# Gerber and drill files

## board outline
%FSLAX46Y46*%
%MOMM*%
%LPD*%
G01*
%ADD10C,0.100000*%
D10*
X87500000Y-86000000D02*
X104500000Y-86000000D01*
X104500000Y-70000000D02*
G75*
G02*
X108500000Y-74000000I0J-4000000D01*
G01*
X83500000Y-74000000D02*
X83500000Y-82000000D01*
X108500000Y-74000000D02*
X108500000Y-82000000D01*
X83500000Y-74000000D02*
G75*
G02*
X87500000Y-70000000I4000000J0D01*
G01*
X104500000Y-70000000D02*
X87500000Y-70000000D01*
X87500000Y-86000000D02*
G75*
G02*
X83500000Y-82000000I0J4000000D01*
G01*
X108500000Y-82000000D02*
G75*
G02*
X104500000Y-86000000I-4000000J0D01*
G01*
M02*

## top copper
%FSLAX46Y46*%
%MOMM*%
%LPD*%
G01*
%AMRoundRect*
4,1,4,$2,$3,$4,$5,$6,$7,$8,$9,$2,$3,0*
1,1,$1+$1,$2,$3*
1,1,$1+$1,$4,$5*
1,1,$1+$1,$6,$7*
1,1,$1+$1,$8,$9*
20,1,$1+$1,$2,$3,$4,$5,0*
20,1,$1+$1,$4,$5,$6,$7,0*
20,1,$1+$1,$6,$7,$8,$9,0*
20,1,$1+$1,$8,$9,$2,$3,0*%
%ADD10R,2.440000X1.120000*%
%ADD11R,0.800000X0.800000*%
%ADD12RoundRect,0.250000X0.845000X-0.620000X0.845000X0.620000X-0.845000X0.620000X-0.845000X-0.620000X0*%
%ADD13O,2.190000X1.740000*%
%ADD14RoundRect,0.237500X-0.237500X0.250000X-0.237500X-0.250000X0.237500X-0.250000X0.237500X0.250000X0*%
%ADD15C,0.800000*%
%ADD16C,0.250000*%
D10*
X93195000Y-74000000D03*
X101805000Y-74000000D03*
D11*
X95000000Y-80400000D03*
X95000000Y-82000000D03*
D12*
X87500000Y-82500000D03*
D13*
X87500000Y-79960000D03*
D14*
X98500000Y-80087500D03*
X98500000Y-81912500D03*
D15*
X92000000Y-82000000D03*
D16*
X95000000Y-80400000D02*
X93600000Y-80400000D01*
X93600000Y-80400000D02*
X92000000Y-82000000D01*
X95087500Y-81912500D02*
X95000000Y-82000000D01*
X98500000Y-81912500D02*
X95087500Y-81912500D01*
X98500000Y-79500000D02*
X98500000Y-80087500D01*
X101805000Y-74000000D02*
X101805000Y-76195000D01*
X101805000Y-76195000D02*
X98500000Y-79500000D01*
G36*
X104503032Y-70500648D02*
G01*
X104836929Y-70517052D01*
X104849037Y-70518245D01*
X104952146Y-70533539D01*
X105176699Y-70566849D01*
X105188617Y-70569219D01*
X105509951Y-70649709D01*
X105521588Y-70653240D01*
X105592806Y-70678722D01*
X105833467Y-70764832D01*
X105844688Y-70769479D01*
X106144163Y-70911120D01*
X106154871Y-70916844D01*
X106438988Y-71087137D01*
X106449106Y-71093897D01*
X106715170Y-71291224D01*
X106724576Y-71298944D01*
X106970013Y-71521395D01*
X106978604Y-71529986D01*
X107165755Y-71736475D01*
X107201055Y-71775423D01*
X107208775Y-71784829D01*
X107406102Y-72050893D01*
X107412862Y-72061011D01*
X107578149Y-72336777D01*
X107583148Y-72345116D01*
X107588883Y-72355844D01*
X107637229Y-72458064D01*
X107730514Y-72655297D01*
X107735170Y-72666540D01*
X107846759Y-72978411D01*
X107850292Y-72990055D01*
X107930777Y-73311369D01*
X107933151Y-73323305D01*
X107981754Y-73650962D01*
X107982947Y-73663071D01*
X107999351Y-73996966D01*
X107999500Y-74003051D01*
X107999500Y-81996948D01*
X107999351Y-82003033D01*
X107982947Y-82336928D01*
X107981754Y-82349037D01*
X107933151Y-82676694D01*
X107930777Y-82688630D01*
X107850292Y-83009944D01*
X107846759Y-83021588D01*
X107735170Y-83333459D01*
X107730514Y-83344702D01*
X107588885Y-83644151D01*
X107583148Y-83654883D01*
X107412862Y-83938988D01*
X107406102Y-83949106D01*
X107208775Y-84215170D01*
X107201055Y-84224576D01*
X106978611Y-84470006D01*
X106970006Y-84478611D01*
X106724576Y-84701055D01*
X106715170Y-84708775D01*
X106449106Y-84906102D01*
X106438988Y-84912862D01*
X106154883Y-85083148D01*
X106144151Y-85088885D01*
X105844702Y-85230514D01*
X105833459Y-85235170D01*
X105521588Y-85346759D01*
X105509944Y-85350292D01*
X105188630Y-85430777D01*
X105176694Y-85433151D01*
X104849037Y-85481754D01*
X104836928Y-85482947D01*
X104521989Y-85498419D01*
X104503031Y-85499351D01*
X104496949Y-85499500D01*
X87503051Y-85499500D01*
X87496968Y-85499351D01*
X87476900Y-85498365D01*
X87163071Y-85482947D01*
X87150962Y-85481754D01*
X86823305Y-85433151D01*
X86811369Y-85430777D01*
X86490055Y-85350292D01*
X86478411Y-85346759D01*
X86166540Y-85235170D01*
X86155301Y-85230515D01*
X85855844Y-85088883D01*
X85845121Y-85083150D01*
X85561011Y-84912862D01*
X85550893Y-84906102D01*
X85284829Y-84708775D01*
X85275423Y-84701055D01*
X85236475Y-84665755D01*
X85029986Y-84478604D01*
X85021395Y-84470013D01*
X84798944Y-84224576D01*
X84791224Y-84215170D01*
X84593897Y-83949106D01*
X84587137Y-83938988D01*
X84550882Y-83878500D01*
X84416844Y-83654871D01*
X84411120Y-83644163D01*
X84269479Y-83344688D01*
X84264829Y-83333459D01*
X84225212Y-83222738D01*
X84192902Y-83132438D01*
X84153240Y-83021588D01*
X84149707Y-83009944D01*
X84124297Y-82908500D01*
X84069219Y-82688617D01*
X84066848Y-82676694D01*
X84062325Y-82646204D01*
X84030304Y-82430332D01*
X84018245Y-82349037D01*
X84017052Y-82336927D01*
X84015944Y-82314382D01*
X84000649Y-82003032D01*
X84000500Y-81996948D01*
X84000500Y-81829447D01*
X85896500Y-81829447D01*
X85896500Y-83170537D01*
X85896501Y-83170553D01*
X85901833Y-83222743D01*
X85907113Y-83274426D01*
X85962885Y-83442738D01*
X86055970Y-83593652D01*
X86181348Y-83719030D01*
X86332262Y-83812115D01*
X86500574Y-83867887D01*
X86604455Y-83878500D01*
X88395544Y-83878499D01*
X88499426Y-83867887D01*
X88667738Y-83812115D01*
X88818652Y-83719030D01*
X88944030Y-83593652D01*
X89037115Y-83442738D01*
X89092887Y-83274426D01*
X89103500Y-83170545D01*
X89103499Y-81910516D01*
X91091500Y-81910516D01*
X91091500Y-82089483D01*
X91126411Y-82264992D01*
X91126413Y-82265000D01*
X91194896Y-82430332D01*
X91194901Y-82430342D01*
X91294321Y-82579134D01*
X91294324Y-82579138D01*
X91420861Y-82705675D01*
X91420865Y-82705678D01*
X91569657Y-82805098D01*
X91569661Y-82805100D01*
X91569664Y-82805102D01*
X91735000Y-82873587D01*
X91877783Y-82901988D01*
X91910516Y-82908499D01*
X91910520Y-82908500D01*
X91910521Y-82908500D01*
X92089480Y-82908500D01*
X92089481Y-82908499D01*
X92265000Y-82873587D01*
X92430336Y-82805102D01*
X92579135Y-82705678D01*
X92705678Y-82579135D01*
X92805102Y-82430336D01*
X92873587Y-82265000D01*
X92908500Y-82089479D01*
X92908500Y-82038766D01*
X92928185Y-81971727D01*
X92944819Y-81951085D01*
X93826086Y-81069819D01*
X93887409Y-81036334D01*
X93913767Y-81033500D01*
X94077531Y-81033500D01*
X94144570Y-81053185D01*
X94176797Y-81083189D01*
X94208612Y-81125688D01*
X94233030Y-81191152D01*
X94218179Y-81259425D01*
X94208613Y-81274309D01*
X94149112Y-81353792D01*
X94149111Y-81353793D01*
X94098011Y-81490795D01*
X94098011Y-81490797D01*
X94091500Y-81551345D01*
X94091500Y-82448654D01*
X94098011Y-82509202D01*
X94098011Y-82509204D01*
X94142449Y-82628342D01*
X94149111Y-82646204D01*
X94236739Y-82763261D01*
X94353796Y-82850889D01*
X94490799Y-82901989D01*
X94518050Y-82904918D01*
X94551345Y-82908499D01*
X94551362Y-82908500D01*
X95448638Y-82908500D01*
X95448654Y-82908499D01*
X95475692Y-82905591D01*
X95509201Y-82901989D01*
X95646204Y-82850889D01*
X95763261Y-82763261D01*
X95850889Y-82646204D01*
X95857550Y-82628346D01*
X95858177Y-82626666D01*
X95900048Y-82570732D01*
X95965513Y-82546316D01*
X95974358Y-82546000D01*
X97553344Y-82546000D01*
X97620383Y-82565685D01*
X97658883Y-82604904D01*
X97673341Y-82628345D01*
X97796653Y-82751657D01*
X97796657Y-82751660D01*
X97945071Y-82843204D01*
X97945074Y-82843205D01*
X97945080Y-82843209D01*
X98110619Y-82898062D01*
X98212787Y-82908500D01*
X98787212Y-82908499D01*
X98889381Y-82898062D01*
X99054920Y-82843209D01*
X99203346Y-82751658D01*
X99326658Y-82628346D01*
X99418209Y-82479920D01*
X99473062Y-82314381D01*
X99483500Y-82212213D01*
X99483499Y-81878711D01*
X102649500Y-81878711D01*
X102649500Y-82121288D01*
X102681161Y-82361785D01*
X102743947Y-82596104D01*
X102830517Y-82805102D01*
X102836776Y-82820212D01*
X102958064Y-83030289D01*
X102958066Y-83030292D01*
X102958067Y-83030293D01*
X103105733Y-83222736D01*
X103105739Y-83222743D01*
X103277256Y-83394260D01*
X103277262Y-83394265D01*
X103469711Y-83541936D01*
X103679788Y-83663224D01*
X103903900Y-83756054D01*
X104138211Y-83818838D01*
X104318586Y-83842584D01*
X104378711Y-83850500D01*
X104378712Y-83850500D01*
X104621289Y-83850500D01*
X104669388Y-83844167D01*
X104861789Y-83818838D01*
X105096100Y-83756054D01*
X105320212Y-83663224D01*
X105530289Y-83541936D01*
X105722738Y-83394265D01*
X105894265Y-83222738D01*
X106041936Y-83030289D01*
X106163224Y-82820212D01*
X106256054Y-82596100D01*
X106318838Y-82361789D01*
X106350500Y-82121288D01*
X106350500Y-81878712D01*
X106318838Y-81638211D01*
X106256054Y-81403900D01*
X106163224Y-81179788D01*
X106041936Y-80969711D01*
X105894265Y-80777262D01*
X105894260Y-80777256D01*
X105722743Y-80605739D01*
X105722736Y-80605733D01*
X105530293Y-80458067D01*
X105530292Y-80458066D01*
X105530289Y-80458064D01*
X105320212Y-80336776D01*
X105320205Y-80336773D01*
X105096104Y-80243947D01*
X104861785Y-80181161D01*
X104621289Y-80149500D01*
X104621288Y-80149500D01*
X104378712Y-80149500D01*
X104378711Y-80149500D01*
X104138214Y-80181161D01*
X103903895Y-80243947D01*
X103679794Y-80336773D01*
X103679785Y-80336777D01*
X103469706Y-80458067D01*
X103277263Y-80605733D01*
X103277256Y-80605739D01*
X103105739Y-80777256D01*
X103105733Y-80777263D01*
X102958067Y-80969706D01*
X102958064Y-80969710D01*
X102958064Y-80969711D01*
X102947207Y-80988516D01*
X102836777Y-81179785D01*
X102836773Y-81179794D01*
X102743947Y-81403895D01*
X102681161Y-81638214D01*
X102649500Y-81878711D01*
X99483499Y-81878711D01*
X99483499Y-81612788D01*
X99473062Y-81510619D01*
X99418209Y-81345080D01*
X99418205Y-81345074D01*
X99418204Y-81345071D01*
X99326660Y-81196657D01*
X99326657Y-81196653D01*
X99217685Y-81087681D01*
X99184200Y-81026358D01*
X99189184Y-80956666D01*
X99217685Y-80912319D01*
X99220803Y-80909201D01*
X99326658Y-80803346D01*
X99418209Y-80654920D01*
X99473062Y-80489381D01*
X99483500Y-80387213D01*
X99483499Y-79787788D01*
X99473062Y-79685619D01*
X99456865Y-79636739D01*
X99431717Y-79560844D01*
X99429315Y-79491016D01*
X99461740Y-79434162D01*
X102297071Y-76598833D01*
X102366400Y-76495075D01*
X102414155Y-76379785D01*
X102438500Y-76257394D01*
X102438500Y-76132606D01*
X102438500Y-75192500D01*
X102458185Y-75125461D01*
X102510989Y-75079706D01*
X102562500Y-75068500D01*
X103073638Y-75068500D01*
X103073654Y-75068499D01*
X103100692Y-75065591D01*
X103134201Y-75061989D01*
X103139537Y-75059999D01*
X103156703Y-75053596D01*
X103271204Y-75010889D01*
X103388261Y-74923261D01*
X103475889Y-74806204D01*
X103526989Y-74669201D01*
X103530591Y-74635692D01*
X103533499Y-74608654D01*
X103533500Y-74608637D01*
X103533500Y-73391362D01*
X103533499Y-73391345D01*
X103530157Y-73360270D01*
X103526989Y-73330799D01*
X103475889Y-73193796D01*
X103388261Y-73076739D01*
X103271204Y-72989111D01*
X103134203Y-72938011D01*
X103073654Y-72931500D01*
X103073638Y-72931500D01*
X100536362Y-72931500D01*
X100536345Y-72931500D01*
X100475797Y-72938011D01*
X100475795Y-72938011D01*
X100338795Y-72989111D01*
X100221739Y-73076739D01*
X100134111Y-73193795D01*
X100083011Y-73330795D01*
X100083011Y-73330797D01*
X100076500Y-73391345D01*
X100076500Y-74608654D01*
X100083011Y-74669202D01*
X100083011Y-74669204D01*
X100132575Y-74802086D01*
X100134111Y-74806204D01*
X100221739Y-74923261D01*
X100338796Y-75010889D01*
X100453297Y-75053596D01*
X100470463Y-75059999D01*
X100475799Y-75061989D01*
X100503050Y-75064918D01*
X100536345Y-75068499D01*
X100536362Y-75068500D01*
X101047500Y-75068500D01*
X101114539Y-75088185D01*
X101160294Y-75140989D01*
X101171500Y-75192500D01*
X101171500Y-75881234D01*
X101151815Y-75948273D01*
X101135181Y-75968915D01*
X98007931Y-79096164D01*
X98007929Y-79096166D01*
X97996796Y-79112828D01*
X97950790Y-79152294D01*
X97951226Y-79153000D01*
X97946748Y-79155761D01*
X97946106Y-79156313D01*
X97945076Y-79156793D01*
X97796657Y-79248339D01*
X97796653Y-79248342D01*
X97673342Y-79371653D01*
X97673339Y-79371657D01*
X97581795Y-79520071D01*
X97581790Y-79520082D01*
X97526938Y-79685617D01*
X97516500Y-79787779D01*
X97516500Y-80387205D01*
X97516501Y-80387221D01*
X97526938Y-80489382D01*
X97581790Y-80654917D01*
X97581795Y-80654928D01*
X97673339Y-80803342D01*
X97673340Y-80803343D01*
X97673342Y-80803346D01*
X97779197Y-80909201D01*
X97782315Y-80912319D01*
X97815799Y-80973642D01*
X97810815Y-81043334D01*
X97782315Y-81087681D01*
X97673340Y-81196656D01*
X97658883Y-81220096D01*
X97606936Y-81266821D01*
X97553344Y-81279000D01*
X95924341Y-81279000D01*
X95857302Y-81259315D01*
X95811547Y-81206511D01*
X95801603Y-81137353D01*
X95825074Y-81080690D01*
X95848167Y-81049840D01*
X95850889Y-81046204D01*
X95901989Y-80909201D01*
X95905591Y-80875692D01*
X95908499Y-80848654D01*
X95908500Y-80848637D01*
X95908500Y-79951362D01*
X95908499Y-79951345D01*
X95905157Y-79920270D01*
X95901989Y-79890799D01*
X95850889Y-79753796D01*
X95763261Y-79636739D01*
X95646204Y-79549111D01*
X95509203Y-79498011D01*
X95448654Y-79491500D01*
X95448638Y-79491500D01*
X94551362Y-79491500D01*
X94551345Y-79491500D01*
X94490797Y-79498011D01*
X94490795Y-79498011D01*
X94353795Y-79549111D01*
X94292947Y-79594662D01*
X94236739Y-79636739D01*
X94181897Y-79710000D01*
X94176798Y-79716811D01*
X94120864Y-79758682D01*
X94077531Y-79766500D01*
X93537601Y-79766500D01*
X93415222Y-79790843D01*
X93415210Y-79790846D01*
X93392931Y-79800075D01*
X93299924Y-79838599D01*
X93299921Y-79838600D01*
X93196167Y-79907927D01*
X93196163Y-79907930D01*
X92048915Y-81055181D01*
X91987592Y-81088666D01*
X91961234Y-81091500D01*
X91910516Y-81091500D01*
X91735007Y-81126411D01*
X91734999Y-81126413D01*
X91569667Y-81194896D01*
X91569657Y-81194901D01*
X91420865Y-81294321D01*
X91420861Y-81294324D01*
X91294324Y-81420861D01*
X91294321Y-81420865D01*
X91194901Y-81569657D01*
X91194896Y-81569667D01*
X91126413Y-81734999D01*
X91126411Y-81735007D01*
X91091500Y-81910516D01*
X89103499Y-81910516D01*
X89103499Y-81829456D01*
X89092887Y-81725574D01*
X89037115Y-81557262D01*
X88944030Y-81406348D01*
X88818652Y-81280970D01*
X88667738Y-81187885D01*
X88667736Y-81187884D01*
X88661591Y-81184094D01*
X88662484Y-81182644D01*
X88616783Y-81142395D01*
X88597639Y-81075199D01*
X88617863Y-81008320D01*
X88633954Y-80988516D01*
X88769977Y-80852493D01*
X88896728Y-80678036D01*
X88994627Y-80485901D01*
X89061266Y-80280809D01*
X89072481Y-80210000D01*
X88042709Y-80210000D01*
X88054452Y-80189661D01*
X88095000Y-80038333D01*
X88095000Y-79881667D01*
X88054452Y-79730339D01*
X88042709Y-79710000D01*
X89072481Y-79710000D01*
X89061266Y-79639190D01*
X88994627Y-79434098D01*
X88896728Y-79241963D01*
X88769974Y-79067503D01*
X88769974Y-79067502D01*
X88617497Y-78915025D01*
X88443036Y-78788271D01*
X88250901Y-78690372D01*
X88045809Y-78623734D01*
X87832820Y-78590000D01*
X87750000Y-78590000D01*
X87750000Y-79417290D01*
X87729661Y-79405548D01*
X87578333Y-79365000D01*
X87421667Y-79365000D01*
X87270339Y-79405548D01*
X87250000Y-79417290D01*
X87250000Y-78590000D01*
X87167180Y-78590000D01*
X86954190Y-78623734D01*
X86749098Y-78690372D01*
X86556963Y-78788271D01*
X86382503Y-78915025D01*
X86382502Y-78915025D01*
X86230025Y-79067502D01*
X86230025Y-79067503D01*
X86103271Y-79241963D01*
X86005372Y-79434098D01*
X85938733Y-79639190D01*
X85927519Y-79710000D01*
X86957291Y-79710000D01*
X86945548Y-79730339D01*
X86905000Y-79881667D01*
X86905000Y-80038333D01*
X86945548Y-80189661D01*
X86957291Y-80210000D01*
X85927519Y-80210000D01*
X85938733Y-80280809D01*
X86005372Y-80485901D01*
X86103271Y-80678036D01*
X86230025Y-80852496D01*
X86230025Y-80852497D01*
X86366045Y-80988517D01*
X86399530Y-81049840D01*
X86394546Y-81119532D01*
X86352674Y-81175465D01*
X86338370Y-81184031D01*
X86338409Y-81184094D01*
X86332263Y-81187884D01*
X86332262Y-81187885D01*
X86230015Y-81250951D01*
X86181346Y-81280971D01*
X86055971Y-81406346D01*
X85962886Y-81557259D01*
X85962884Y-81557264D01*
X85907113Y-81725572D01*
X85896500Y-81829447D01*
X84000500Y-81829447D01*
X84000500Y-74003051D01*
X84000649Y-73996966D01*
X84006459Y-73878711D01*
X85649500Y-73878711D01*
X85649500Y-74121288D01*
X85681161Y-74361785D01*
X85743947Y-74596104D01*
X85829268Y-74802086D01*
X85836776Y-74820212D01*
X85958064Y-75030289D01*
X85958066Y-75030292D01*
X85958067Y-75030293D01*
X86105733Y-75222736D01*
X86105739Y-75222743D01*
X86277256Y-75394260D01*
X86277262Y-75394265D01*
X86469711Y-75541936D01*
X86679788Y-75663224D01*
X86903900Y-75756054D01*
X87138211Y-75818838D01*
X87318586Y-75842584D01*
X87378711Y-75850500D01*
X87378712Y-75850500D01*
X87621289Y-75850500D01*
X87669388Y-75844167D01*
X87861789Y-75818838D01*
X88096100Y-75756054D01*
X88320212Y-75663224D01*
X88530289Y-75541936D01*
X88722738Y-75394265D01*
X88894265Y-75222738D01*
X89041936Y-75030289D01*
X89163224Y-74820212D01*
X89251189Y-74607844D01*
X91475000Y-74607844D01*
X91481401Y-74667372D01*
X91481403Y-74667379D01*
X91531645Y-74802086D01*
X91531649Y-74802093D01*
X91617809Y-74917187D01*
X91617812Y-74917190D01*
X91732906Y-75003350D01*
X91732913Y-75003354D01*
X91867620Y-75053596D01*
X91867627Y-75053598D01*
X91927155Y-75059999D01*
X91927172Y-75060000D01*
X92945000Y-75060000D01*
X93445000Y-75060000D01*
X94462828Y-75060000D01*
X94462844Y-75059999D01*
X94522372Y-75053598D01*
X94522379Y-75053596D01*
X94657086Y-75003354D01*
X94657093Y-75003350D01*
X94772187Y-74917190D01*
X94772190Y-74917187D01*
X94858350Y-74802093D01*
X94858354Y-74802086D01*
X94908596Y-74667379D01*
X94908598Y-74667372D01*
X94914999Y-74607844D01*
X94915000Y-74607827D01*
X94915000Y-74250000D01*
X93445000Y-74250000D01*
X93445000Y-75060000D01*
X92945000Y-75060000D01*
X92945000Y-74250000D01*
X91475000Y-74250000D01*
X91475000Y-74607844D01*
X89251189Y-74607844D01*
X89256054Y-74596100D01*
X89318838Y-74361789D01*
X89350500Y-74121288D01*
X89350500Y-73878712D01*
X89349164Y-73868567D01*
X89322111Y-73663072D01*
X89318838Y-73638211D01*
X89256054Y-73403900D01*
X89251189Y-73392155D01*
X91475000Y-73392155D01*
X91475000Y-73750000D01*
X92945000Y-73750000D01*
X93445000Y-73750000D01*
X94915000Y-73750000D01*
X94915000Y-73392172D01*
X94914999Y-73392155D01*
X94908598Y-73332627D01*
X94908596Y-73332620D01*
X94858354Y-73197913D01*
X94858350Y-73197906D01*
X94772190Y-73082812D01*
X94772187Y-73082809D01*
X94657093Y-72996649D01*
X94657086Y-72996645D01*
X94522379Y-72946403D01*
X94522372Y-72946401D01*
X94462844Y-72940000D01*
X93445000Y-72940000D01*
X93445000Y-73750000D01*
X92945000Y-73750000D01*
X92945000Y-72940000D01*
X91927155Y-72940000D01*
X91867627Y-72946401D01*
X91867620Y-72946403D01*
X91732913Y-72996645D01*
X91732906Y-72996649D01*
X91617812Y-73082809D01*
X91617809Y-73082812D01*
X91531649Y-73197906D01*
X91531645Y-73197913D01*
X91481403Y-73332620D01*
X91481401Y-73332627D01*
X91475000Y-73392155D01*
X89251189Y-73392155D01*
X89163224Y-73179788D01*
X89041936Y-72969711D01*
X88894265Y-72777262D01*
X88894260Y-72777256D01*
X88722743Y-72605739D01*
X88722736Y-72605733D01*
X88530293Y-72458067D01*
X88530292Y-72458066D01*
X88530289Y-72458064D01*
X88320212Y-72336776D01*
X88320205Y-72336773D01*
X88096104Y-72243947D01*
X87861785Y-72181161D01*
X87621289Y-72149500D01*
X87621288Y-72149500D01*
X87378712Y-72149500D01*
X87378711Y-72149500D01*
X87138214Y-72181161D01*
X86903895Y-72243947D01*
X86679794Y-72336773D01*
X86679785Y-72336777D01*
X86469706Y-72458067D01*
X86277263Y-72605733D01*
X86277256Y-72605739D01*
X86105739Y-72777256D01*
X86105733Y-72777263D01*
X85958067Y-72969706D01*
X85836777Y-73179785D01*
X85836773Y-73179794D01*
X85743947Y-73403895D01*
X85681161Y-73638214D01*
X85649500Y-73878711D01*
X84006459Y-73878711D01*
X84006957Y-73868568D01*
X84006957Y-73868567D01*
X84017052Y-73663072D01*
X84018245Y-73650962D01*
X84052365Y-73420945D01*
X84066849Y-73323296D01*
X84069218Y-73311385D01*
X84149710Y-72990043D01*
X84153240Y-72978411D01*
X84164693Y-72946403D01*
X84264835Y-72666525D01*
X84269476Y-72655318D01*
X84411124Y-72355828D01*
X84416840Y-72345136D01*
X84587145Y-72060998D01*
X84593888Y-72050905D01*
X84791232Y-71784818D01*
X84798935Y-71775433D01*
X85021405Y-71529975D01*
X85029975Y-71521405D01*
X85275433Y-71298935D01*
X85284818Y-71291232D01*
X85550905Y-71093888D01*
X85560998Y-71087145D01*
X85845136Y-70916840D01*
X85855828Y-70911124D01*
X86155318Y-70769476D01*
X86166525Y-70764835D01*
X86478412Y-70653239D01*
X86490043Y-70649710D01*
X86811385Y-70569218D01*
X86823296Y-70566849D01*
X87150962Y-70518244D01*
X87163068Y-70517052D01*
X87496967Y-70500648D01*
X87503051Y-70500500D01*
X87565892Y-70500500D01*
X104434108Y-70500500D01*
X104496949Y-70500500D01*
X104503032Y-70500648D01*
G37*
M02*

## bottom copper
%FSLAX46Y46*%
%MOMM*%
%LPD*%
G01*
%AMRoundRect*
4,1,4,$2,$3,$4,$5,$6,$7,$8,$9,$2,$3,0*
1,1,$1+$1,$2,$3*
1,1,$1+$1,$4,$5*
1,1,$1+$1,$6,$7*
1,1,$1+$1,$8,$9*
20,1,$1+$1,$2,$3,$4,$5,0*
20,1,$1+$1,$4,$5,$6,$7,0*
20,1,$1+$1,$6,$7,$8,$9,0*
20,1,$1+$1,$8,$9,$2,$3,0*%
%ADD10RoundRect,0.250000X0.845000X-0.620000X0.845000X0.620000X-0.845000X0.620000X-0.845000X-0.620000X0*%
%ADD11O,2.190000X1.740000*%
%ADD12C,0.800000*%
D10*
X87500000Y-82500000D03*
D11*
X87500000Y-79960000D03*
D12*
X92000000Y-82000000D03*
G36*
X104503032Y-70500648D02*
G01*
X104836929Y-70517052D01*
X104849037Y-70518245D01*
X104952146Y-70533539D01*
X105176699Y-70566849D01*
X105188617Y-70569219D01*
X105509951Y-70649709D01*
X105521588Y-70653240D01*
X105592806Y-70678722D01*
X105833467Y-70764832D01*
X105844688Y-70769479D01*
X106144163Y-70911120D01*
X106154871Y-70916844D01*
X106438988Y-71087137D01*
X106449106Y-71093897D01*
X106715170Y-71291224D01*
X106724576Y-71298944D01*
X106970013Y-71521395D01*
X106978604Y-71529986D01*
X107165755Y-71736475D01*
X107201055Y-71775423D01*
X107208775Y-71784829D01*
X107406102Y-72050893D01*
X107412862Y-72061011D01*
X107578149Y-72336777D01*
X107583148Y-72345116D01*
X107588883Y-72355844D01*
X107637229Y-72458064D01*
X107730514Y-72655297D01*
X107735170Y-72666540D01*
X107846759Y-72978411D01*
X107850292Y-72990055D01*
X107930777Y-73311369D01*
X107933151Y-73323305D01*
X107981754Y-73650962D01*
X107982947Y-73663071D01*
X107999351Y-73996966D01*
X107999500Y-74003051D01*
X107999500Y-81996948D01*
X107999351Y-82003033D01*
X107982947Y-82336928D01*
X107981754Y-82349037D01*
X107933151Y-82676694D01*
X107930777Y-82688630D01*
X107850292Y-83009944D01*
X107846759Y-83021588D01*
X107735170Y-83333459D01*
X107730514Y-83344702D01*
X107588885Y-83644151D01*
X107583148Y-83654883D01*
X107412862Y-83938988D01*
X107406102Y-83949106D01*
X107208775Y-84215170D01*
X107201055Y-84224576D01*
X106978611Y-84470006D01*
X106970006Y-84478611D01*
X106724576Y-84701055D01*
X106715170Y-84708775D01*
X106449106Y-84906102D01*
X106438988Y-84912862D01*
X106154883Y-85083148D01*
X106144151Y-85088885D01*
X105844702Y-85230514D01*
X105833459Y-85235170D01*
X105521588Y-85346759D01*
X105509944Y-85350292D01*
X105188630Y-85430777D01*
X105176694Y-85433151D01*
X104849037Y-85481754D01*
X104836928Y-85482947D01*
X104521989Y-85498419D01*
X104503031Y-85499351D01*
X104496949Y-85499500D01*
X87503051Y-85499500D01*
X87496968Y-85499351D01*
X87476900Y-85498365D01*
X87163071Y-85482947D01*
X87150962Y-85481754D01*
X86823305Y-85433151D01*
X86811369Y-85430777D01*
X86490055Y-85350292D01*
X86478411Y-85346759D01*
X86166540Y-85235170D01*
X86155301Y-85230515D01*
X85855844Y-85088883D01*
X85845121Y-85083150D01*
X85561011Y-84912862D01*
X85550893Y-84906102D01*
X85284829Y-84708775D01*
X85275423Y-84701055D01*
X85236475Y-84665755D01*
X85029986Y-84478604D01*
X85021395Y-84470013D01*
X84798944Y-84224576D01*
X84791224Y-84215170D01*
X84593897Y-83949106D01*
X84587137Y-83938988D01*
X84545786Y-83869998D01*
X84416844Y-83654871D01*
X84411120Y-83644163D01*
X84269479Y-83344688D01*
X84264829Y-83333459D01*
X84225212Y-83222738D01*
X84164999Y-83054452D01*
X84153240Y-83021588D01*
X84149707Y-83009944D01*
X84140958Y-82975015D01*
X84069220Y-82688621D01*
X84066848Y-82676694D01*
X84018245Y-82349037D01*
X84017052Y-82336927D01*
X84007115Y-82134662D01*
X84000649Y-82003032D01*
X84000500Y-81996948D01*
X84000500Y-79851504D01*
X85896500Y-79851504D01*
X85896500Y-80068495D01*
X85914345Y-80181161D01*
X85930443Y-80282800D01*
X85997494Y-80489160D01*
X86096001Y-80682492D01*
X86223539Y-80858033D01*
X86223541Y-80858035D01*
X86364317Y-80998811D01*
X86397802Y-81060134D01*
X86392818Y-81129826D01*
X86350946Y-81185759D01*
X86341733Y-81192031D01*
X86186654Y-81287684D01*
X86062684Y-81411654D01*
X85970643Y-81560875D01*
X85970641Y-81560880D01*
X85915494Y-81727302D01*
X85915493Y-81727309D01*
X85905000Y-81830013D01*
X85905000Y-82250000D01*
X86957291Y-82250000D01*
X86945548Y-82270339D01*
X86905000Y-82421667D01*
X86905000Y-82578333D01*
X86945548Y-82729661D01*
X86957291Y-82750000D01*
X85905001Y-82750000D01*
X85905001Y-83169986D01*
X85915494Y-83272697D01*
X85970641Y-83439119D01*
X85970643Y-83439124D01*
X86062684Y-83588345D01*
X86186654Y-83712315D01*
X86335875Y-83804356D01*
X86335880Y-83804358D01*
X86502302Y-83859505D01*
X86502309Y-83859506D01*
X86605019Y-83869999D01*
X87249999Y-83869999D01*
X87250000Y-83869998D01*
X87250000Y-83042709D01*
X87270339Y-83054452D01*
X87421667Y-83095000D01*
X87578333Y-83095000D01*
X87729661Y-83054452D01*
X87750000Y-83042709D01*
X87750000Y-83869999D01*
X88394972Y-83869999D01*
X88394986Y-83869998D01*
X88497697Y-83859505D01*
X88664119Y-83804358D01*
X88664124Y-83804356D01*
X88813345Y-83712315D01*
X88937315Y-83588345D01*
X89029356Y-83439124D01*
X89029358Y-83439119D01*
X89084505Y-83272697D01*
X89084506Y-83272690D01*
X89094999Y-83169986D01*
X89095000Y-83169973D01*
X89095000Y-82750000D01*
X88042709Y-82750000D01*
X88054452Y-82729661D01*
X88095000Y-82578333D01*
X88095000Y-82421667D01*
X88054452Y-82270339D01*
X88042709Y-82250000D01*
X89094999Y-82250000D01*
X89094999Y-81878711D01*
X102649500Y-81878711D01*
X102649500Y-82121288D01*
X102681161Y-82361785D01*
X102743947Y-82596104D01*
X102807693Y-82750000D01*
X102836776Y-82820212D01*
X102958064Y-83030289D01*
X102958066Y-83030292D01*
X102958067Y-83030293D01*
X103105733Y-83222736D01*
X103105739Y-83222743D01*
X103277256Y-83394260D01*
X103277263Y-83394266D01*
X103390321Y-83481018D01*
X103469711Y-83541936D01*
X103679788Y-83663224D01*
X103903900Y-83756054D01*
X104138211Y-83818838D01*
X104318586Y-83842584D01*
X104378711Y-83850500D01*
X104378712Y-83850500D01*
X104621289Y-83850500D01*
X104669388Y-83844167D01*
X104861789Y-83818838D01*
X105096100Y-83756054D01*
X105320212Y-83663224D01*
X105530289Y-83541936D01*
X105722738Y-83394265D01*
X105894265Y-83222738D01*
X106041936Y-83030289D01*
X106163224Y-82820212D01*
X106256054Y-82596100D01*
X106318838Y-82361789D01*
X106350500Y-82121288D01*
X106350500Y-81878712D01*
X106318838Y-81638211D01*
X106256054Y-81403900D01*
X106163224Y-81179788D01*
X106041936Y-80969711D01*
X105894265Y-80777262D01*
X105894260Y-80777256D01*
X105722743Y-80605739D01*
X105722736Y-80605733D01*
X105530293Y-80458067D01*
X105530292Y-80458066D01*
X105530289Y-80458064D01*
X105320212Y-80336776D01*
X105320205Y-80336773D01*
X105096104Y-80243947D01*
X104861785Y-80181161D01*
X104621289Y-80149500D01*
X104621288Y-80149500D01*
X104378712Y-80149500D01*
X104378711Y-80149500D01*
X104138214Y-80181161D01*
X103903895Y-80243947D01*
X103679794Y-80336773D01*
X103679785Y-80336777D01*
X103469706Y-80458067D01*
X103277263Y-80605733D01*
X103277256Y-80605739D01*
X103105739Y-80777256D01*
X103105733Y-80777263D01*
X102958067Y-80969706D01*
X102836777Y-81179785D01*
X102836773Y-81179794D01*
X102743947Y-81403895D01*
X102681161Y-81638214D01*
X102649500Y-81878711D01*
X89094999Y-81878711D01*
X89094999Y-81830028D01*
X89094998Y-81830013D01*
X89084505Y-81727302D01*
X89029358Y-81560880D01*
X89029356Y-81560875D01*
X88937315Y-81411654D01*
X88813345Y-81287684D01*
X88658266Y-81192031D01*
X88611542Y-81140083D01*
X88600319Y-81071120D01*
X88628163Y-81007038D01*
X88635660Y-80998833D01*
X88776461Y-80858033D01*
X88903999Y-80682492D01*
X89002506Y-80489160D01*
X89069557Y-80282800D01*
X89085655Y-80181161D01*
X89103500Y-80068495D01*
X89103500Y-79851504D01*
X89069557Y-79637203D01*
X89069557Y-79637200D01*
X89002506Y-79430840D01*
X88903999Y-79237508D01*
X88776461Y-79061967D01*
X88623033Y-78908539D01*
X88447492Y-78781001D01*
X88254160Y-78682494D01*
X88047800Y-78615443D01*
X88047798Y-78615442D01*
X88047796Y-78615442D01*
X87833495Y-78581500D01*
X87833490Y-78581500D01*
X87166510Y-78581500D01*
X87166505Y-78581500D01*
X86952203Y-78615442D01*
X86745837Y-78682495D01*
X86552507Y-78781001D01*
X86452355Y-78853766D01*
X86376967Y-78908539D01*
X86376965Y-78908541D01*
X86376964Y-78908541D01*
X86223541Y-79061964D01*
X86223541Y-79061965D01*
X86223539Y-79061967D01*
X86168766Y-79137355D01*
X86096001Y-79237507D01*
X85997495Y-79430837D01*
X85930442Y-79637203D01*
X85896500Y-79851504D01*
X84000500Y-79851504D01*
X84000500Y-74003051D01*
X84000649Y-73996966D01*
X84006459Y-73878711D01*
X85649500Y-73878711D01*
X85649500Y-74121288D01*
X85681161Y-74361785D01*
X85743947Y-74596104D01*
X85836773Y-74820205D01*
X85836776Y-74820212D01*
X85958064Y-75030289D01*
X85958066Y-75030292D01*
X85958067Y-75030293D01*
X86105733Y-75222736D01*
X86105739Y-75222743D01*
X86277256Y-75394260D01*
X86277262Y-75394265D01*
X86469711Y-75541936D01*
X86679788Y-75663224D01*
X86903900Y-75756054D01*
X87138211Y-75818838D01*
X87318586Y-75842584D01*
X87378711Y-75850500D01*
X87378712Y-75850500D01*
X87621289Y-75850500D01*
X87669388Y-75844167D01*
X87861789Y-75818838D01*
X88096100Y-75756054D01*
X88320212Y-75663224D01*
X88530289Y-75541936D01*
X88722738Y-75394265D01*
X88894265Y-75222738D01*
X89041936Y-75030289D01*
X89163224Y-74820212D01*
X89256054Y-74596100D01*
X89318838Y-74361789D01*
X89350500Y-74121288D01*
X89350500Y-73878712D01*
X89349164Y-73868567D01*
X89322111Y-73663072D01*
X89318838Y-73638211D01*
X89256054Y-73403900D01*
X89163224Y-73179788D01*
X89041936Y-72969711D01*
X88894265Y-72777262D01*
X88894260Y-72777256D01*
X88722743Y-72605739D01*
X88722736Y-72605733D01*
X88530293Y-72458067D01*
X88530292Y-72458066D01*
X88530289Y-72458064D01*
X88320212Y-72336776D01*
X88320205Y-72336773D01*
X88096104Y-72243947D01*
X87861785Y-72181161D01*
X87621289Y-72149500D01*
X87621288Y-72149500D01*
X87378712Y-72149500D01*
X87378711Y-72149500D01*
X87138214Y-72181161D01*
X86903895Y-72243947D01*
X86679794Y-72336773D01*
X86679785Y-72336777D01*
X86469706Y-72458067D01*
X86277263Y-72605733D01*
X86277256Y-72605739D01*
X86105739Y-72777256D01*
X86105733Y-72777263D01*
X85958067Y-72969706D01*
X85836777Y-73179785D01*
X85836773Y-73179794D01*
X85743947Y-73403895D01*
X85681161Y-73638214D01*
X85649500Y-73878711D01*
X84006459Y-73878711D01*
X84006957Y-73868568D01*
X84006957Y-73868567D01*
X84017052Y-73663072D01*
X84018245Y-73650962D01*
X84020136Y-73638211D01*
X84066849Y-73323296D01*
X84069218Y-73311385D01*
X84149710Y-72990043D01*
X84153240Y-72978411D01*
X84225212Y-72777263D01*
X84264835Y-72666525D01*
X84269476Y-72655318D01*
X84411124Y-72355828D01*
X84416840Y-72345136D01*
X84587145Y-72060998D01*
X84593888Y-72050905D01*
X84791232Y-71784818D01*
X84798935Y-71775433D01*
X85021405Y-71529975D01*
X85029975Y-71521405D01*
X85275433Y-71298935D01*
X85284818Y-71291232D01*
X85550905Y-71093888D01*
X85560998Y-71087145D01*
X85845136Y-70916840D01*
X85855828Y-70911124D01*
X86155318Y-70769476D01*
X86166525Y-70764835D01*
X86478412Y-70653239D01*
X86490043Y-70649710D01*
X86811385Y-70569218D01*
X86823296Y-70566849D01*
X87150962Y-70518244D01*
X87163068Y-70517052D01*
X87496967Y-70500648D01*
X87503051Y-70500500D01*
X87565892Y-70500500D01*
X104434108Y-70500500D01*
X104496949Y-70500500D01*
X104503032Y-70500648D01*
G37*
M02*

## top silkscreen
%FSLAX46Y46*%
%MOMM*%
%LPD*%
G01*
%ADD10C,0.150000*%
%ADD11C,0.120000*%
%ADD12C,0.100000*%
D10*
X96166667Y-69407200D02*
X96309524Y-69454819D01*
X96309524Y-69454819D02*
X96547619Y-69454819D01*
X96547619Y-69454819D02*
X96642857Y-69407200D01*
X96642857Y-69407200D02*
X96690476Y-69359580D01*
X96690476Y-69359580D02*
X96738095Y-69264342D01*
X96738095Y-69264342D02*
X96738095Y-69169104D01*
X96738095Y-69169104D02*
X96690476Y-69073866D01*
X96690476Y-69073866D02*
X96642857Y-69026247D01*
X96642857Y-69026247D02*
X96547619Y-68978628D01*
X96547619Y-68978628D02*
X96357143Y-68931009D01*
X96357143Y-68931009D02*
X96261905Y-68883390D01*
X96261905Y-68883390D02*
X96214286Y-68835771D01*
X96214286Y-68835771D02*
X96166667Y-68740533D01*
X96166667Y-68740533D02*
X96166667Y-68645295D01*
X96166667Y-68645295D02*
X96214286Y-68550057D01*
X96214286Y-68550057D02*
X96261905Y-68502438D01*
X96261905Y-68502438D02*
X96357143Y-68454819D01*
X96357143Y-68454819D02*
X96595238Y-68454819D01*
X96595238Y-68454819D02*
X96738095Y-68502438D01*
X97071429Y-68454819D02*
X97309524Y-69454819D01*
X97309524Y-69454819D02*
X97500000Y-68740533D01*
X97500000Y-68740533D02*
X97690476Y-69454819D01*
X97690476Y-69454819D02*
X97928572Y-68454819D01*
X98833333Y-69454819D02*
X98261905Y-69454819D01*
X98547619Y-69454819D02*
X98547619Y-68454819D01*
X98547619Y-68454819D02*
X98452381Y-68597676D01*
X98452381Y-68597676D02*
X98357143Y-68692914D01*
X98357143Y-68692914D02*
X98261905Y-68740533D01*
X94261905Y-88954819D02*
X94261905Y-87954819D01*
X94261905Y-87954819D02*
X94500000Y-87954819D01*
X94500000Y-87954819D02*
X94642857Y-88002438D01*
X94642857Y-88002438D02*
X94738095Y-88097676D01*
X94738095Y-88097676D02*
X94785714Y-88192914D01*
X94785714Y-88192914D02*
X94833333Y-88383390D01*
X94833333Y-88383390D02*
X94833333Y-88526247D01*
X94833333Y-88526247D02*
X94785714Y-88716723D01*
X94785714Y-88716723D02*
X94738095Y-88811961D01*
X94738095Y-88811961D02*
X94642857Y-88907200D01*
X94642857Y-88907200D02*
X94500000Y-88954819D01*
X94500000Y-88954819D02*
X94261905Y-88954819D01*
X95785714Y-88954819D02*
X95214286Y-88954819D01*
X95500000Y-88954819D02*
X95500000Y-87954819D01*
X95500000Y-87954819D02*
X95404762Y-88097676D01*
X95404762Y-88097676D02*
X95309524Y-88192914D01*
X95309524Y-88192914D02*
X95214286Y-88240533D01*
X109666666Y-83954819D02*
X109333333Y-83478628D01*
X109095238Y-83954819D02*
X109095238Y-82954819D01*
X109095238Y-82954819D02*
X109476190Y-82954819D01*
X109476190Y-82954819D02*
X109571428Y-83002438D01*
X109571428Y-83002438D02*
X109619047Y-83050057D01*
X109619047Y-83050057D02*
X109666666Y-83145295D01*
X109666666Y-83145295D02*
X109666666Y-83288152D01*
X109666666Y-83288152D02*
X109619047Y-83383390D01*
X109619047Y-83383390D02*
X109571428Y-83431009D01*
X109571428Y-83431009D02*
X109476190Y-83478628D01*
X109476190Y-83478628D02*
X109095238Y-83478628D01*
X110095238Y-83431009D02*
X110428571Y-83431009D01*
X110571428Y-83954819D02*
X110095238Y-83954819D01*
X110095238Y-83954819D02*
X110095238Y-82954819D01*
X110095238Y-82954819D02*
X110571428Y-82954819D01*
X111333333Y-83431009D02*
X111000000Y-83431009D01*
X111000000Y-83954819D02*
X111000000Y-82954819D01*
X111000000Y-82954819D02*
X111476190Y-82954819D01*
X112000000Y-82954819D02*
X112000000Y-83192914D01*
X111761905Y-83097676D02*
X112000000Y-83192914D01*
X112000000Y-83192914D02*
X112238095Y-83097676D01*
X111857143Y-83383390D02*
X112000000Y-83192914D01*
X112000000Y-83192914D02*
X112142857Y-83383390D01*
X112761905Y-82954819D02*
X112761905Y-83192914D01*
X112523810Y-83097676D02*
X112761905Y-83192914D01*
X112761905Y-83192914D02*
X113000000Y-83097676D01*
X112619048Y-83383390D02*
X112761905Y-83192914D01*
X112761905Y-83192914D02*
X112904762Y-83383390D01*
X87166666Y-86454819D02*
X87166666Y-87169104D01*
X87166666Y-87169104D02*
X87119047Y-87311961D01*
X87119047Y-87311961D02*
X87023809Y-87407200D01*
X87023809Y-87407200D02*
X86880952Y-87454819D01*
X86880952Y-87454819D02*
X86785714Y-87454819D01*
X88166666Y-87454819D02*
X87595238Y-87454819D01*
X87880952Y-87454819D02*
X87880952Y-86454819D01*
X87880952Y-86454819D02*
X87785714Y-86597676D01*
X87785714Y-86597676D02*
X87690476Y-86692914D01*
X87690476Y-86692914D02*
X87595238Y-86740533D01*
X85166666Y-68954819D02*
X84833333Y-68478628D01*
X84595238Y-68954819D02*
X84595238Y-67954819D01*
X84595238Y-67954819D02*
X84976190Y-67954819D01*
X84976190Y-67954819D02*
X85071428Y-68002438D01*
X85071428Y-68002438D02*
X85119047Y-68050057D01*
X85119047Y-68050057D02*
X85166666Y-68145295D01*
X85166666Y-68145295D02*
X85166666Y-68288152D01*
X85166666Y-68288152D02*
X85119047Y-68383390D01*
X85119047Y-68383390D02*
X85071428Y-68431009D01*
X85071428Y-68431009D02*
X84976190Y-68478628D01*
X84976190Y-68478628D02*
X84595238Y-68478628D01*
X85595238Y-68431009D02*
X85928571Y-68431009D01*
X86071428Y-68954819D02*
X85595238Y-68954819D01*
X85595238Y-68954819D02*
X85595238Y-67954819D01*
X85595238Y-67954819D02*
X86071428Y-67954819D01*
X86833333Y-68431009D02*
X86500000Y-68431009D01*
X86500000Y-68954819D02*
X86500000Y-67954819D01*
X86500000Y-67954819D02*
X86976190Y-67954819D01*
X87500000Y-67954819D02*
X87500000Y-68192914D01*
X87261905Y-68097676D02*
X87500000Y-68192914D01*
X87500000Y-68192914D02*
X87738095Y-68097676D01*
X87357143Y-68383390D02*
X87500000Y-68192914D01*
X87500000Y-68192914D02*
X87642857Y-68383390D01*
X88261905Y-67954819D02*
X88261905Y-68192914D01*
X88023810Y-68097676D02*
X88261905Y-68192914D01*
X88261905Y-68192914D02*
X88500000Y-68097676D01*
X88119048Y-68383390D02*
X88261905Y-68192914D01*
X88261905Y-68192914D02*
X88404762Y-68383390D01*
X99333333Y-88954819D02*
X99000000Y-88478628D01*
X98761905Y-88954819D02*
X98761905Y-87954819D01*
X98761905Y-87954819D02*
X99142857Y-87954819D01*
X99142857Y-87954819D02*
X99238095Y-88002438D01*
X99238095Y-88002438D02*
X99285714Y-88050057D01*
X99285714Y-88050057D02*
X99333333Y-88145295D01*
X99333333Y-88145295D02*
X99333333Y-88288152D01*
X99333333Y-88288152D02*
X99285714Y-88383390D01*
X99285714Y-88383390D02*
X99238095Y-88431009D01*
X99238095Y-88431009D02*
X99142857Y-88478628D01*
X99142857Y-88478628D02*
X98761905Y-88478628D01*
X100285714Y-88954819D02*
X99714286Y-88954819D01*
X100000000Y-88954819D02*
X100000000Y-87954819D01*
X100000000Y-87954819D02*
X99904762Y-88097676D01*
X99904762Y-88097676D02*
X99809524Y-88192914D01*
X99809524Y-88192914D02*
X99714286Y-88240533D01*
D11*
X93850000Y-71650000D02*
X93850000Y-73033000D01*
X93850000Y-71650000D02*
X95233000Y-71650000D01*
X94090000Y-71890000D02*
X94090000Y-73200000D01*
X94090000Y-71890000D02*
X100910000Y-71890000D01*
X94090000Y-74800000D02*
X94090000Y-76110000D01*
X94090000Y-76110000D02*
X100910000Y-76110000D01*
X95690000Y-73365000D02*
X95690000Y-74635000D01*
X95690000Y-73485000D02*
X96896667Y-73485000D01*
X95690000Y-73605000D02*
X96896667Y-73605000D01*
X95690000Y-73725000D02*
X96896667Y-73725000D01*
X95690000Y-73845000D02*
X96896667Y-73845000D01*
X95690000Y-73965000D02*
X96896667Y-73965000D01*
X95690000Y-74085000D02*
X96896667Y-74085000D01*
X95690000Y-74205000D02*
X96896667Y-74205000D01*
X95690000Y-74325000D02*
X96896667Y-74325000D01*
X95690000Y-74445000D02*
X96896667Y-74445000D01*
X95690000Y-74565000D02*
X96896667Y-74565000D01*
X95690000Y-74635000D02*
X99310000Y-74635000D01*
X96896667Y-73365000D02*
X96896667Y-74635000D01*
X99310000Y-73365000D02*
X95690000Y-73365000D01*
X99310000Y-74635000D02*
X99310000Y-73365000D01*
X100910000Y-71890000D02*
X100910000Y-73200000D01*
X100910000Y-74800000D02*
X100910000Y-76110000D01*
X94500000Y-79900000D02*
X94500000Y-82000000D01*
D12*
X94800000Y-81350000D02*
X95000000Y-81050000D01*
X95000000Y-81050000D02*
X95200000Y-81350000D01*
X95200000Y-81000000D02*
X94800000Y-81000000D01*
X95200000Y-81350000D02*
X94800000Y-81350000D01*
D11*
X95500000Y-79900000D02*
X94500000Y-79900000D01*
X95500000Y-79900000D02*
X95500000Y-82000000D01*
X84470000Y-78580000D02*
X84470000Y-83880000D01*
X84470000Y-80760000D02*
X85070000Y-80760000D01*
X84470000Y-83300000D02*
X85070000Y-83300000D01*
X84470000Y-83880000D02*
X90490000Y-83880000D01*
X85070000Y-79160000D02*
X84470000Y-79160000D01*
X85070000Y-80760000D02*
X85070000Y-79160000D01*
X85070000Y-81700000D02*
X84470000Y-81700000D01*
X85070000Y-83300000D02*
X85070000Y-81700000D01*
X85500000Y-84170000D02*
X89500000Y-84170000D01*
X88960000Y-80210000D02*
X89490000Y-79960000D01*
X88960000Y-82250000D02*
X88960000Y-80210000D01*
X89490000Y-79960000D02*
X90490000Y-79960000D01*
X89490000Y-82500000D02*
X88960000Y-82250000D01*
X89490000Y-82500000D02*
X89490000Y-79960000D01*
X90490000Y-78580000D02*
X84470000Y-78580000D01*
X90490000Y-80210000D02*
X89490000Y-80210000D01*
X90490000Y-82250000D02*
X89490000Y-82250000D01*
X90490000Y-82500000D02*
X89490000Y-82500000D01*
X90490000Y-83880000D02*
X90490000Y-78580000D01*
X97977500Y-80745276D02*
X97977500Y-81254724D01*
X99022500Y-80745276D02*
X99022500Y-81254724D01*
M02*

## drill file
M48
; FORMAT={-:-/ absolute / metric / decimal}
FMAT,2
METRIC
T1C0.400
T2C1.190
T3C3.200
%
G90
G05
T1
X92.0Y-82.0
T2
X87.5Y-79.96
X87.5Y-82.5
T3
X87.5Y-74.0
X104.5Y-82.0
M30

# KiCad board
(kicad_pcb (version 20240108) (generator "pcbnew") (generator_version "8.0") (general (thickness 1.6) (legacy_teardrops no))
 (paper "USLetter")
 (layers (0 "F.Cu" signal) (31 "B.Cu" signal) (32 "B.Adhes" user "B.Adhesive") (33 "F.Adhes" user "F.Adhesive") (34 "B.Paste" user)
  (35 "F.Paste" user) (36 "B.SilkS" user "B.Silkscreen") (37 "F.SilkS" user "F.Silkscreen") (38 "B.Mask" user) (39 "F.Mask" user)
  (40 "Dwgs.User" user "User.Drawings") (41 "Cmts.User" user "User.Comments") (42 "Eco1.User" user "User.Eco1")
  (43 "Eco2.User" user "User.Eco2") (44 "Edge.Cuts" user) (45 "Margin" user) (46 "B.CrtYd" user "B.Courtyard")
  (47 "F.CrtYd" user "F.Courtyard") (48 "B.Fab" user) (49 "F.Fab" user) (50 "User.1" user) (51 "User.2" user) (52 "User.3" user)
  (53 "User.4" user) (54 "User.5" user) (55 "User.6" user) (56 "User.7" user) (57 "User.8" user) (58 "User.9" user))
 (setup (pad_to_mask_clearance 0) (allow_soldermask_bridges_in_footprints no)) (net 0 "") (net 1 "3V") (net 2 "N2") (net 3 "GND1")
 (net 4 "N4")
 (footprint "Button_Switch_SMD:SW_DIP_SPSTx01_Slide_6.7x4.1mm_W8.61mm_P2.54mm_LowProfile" (layer "F.Cu") (at 97.5 74)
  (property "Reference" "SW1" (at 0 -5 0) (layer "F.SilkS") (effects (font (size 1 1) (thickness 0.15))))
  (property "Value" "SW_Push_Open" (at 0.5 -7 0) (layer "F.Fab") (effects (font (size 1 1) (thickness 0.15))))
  (fp_line (start -3.65 -2.35) (end -3.65 -0.967) (stroke (width 0.12) (type solid)) (layer "F.SilkS"))
  (fp_line (start -3.65 -2.35) (end -2.267 -2.35) (stroke (width 0.12) (type solid)) (layer "F.SilkS"))
  (fp_line (start -3.41 -2.11) (end -3.41 -0.8) (stroke (width 0.12) (type solid)) (layer "F.SilkS"))
  (fp_line (start -3.41 -2.11) (end 3.41 -2.11) (stroke (width 0.12) (type solid)) (layer "F.SilkS"))
  (fp_line (start -3.41 0.8) (end -3.41 2.11) (stroke (width 0.12) (type solid)) (layer "F.SilkS"))
  (fp_line (start -3.41 2.11) (end 3.41 2.11) (stroke (width 0.12) (type solid)) (layer "F.SilkS"))
  (fp_line (start -1.81 -0.635) (end -1.81 0.635) (stroke (width 0.12) (type solid)) (layer "F.SilkS"))
  (fp_line (start -1.81 -0.515) (end -0.603333 -0.515) (stroke (width 0.12) (type solid)) (layer "F.SilkS"))
  (fp_line (start -1.81 -0.395) (end -0.603333 -0.395) (stroke (width 0.12) (type solid)) (layer "F.SilkS"))
  (fp_line (start -1.81 -0.275) (end -0.603333 -0.275) (stroke (width 0.12) (type solid)) (layer "F.SilkS"))
  (fp_line (start -1.81 -0.155) (end -0.603333 -0.155) (stroke (width 0.12) (type solid)) (layer "F.SilkS"))
  (fp_line (start -1.81 -0.035) (end -0.603333 -0.035) (stroke (width 0.12) (type solid)) (layer "F.SilkS"))
  (fp_line (start -1.81 0.085) (end -0.603333 0.085) (stroke (width 0.12) (type solid)) (layer "F.SilkS"))
  (fp_line (start -1.81 0.205) (end -0.603333 0.205) (stroke (width 0.12) (type solid)) (layer "F.SilkS"))
  (fp_line (start -1.81 0.325) (end -0.603333 0.325) (stroke (width 0.12) (type solid)) (layer "F.SilkS"))
  (fp_line (start -1.81 0.445) (end -0.603333 0.445) (stroke (width 0.12) (type solid)) (layer "F.SilkS"))
  (fp_line (start -1.81 0.565) (end -0.603333 0.565) (stroke (width 0.12) (type solid)) (layer "F.SilkS"))
  (fp_line (start -1.81 0.635) (end 1.81 0.635) (stroke (width 0.12) (type solid)) (layer "F.SilkS"))
  (fp_line (start -0.603333 -0.635) (end -0.603333 0.635) (stroke (width 0.12) (type solid)) (layer "F.SilkS"))
  (fp_line (start 1.81 -0.635) (end -1.81 -0.635) (stroke (width 0.12) (type solid)) (layer "F.SilkS"))
  (fp_line (start 1.81 0.635) (end 1.81 -0.635) (stroke (width 0.12) (type solid)) (layer "F.SilkS"))
  (fp_line (start 3.41 -2.11) (end 3.41 -0.8) (stroke (width 0.12) (type solid)) (layer "F.SilkS"))
  (fp_line (start 3.41 0.8) (end 3.41 2.11) (stroke (width 0.12) (type solid)) (layer "F.SilkS"))
  (pad "1" smd rect (at -4.305 0) (size 2.44 1.12) (layers "F.Cu" "F.Paste" "F.Mask") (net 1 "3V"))
  (pad "2" smd rect (at 4.305 0) (size 2.44 1.12) (layers "F.Cu" "F.Paste" "F.Mask") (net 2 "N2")))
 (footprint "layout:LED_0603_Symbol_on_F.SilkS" (layer "F.Cu") (at 95 81.2 -90)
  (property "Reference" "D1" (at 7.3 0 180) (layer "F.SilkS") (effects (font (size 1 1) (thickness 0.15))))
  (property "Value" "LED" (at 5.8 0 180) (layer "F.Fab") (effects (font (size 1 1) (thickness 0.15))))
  (fp_line (start -1.3 0.5) (end 0.8 0.5) (stroke (width 0.12) (type solid)) (layer "F.SilkS"))
  (fp_line (start 0.15 0.2) (end -0.15 0) (stroke (width 0.1) (type solid)) (layer "F.SilkS"))
  (fp_line (start -0.15 0) (end 0.15 -0.2) (stroke (width 0.1) (type solid)) (layer "F.SilkS"))
  (fp_line (start -0.2 -0.2) (end -0.2 0.2) (stroke (width 0.1) (type solid)) (layer "F.SilkS"))
  (fp_line (start 0.15 -0.2) (end 0.15 0.2) (stroke (width 0.1) (type solid)) (layer "F.SilkS"))
  (fp_line (start -1.3 -0.5) (end -1.3 0.5) (stroke (width 0.12) (type solid)) (layer "F.SilkS"))
  (fp_line (start -1.3 -0.5) (end 0.8 -0.5) (stroke (width 0.12) (type solid)) (layer "F.SilkS"))
  (pad "1" smd rect (at -0.8 0 90) (size 0.8 0.8) (layers "F.Cu" "F.Paste" "F.Mask") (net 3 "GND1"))
  (pad "2" smd rect (at 0.8 0 90) (size 0.8 0.8) (layers "F.Cu" "F.Paste" "F.Mask") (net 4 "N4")))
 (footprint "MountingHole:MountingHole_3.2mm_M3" (layer "F.Cu") (at 104.5 82)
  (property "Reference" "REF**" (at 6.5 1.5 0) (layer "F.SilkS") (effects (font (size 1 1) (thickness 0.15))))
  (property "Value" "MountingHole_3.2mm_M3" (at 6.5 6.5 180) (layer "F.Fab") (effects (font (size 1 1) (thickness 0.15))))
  (pad "" np_thru_hole circle (at 0 0) (size 3.2 3.2) (drill 3.2) (layers "*.Cu" "*.Mask")))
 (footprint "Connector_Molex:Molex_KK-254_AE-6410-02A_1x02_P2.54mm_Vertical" (layer "F.Cu") (at 87.5 82.5 90)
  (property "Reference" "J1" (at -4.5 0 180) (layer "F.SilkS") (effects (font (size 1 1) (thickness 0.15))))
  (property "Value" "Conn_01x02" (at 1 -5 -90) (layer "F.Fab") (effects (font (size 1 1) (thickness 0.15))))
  (fp_line (start 3.92 -3.03) (end -1.38 -3.03) (stroke (width 0.12) (type solid)) (layer "F.SilkS"))
  (fp_line (start 1.74 -3.03) (end 1.74 -2.43) (stroke (width 0.12) (type solid)) (layer "F.SilkS"))
  (fp_line (start -0.8 -3.03) (end -0.8 -2.43) (stroke (width 0.12) (type solid)) (layer "F.SilkS"))
  (fp_line (start -1.38 -3.03) (end -1.38 2.99) (stroke (width 0.12) (type solid)) (layer "F.SilkS"))
  (fp_line (start 3.34 -2.43) (end 3.34 -3.03) (stroke (width 0.12) (type solid)) (layer "F.SilkS"))
  (fp_line (start 1.74 -2.43) (end 3.34 -2.43) (stroke (width 0.12) (type solid)) (layer "F.SilkS"))
  (fp_line (start 0.8 -2.43) (end 0.8 -3.03) (stroke (width 0.12) (type solid)) (layer "F.SilkS"))
  (fp_line (start -0.8 -2.43) (end 0.8 -2.43) (stroke (width 0.12) (type solid)) (layer "F.SilkS"))
  (fp_line (start -1.67 -2) (end -1.67 2) (stroke (width 0.12) (type solid)) (layer "F.SilkS"))
  (fp_line (start 2.29 1.46) (end 2.54 1.99) (stroke (width 0.12) (type solid)) (layer "F.SilkS"))
  (fp_line (start 0.25 1.46) (end 2.29 1.46) (stroke (width 0.12) (type solid)) (layer "F.SilkS"))
  (fp_line (start 2.54 1.99) (end 2.54 2.99) (stroke (width 0.12) (type solid)) (layer "F.SilkS"))
  (fp_line (start 0 1.99) (end 0.25 1.46) (stroke (width 0.12) (type solid)) (layer "F.SilkS"))
  (fp_line (start 0 1.99) (end 2.54 1.99) (stroke (width 0.12) (type solid)) (layer "F.SilkS"))
  (fp_line (start 3.92 2.99) (end 3.92 -3.03) (stroke (width 0.12) (type solid)) (layer "F.SilkS"))
  (fp_line (start 2.29 2.99) (end 2.29 1.99) (stroke (width 0.12) (type solid)) (layer "F.SilkS"))
  (fp_line (start 0.25 2.99) (end 0.25 1.99) (stroke (width 0.12) (type solid)) (layer "F.SilkS"))
  (fp_line (start 0 2.99) (end 0 1.99) (stroke (width 0.12) (type solid)) (layer "F.SilkS"))
  (fp_line (start -1.38 2.99) (end 3.92 2.99) (stroke (width 0.12) (type solid)) (layer "F.SilkS"))
  (pad "1" thru_hole roundrect (at 0 0 90) (size 1.74 2.19) (drill 1.19) (layers "*.Cu" "*.Mask") (remove_unused_layers no)
   (roundrect_rratio 0.143678) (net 3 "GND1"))
  (pad "2" thru_hole oval (at 2.54 0 90) (size 1.74 2.19) (drill 1.19) (layers "*.Cu" "*.Mask") (remove_unused_layers no) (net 1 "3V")))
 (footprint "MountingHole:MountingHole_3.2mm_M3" (layer "F.Cu") (at 87.5 74)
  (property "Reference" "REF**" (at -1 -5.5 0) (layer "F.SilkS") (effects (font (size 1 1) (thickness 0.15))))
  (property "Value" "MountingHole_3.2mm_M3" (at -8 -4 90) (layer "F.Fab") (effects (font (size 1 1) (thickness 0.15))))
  (pad "" np_thru_hole circle (at 0 0) (size 3.2 3.2) (drill 3.2) (layers "*.Cu" "*.Mask")))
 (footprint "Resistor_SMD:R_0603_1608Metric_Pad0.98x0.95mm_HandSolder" (layer "F.Cu") (at 98.5 81 -90)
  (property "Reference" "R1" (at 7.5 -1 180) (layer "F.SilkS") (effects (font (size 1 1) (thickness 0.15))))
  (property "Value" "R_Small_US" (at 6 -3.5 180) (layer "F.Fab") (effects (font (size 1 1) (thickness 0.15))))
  (fp_line (start -0.254724 0.5225) (end 0.254724 0.5225) (stroke (width 0.12) (type solid)) (layer "F.SilkS"))
  (fp_line (start -0.254724 -0.5225) (end 0.254724 -0.5225) (stroke (width 0.12) (type solid)) (layer "F.SilkS"))
  (pad "1" smd roundrect (at -0.9125 0 270) (size 0.975 0.95) (layers "F.Cu" "F.Paste" "F.Mask") (roundrect_rratio 0.25) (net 2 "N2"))
  (pad "2" smd roundrect (at 0.9125 0 270) (size 0.975 0.95) (layers "F.Cu" "F.Paste" "F.Mask") (roundrect_rratio 0.25) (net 4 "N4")))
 (gr_line (start 87.5 86) (end 104.5 86) (stroke (width 0.1) (type default)) (layer "Edge.Cuts"))
 (gr_arc (start 104.5 70) (mid 107.328427 71.171573) (end 108.5 74) (stroke (width 0.1) (type default)) (layer "Edge.Cuts"))
 (gr_line (start 83.5 74) (end 83.5 82) (stroke (width 0.1) (type default)) (layer "Edge.Cuts"))
 (gr_line (start 108.5 74) (end 108.5 82) (stroke (width 0.1) (type default)) (layer "Edge.Cuts"))
 (gr_arc (start 83.5 74) (mid 84.671573 71.171573) (end 87.5 70) (stroke (width 0.1) (type default)) (layer "Edge.Cuts"))
 (gr_line (start 104.5 70) (end 87.5 70) (stroke (width 0.1) (type default)) (layer "Edge.Cuts"))
 (gr_arc (start 87.5 86) (mid 84.671573 84.828427) (end 83.5 82) (stroke (width 0.1) (type default)) (layer "Edge.Cuts"))
 (gr_arc (start 108.5 82) (mid 107.328427 84.828427) (end 104.5 86) (stroke (width 0.1) (type default)) (layer "Edge.Cuts"))
 (segment (start 95 80.4) (end 93.6 80.4) (width 0.25) (layer "F.Cu") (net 3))
 (segment (start 93.6 80.4) (end 92 82) (width 0.25) (layer "F.Cu") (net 3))
 (via (at 92 82) (size 0.8) (drill 0.4) (layers "F.Cu" "B.Cu") (free yes) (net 3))
 (segment (start 95.0875 81.9125) (end 95 82) (width 0.25) (layer "F.Cu") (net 4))
 (segment (start 98.5 81.9125) (end 95.0875 81.9125) (width 0.25) (layer "F.Cu") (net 4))
 (segment (start 98.5 79.5) (end 98.5 80.0875) (width 0.25) (layer "F.Cu") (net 2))
 (segment (start 101.805 74) (end 101.805 76.195) (width 0.25) (layer "F.Cu") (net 2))
 (segment (start 101.805 76.195) (end 98.5 79.5) (width 0.25) (layer "F.Cu") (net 2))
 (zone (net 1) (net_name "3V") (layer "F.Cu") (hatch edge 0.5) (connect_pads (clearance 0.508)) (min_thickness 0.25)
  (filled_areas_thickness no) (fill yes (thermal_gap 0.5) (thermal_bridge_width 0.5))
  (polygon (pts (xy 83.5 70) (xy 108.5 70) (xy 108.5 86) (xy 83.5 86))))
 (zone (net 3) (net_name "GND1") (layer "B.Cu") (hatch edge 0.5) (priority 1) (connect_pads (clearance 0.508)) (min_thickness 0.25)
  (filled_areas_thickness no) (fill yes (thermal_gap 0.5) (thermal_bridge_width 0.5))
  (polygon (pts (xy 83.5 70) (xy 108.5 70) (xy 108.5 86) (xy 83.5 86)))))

